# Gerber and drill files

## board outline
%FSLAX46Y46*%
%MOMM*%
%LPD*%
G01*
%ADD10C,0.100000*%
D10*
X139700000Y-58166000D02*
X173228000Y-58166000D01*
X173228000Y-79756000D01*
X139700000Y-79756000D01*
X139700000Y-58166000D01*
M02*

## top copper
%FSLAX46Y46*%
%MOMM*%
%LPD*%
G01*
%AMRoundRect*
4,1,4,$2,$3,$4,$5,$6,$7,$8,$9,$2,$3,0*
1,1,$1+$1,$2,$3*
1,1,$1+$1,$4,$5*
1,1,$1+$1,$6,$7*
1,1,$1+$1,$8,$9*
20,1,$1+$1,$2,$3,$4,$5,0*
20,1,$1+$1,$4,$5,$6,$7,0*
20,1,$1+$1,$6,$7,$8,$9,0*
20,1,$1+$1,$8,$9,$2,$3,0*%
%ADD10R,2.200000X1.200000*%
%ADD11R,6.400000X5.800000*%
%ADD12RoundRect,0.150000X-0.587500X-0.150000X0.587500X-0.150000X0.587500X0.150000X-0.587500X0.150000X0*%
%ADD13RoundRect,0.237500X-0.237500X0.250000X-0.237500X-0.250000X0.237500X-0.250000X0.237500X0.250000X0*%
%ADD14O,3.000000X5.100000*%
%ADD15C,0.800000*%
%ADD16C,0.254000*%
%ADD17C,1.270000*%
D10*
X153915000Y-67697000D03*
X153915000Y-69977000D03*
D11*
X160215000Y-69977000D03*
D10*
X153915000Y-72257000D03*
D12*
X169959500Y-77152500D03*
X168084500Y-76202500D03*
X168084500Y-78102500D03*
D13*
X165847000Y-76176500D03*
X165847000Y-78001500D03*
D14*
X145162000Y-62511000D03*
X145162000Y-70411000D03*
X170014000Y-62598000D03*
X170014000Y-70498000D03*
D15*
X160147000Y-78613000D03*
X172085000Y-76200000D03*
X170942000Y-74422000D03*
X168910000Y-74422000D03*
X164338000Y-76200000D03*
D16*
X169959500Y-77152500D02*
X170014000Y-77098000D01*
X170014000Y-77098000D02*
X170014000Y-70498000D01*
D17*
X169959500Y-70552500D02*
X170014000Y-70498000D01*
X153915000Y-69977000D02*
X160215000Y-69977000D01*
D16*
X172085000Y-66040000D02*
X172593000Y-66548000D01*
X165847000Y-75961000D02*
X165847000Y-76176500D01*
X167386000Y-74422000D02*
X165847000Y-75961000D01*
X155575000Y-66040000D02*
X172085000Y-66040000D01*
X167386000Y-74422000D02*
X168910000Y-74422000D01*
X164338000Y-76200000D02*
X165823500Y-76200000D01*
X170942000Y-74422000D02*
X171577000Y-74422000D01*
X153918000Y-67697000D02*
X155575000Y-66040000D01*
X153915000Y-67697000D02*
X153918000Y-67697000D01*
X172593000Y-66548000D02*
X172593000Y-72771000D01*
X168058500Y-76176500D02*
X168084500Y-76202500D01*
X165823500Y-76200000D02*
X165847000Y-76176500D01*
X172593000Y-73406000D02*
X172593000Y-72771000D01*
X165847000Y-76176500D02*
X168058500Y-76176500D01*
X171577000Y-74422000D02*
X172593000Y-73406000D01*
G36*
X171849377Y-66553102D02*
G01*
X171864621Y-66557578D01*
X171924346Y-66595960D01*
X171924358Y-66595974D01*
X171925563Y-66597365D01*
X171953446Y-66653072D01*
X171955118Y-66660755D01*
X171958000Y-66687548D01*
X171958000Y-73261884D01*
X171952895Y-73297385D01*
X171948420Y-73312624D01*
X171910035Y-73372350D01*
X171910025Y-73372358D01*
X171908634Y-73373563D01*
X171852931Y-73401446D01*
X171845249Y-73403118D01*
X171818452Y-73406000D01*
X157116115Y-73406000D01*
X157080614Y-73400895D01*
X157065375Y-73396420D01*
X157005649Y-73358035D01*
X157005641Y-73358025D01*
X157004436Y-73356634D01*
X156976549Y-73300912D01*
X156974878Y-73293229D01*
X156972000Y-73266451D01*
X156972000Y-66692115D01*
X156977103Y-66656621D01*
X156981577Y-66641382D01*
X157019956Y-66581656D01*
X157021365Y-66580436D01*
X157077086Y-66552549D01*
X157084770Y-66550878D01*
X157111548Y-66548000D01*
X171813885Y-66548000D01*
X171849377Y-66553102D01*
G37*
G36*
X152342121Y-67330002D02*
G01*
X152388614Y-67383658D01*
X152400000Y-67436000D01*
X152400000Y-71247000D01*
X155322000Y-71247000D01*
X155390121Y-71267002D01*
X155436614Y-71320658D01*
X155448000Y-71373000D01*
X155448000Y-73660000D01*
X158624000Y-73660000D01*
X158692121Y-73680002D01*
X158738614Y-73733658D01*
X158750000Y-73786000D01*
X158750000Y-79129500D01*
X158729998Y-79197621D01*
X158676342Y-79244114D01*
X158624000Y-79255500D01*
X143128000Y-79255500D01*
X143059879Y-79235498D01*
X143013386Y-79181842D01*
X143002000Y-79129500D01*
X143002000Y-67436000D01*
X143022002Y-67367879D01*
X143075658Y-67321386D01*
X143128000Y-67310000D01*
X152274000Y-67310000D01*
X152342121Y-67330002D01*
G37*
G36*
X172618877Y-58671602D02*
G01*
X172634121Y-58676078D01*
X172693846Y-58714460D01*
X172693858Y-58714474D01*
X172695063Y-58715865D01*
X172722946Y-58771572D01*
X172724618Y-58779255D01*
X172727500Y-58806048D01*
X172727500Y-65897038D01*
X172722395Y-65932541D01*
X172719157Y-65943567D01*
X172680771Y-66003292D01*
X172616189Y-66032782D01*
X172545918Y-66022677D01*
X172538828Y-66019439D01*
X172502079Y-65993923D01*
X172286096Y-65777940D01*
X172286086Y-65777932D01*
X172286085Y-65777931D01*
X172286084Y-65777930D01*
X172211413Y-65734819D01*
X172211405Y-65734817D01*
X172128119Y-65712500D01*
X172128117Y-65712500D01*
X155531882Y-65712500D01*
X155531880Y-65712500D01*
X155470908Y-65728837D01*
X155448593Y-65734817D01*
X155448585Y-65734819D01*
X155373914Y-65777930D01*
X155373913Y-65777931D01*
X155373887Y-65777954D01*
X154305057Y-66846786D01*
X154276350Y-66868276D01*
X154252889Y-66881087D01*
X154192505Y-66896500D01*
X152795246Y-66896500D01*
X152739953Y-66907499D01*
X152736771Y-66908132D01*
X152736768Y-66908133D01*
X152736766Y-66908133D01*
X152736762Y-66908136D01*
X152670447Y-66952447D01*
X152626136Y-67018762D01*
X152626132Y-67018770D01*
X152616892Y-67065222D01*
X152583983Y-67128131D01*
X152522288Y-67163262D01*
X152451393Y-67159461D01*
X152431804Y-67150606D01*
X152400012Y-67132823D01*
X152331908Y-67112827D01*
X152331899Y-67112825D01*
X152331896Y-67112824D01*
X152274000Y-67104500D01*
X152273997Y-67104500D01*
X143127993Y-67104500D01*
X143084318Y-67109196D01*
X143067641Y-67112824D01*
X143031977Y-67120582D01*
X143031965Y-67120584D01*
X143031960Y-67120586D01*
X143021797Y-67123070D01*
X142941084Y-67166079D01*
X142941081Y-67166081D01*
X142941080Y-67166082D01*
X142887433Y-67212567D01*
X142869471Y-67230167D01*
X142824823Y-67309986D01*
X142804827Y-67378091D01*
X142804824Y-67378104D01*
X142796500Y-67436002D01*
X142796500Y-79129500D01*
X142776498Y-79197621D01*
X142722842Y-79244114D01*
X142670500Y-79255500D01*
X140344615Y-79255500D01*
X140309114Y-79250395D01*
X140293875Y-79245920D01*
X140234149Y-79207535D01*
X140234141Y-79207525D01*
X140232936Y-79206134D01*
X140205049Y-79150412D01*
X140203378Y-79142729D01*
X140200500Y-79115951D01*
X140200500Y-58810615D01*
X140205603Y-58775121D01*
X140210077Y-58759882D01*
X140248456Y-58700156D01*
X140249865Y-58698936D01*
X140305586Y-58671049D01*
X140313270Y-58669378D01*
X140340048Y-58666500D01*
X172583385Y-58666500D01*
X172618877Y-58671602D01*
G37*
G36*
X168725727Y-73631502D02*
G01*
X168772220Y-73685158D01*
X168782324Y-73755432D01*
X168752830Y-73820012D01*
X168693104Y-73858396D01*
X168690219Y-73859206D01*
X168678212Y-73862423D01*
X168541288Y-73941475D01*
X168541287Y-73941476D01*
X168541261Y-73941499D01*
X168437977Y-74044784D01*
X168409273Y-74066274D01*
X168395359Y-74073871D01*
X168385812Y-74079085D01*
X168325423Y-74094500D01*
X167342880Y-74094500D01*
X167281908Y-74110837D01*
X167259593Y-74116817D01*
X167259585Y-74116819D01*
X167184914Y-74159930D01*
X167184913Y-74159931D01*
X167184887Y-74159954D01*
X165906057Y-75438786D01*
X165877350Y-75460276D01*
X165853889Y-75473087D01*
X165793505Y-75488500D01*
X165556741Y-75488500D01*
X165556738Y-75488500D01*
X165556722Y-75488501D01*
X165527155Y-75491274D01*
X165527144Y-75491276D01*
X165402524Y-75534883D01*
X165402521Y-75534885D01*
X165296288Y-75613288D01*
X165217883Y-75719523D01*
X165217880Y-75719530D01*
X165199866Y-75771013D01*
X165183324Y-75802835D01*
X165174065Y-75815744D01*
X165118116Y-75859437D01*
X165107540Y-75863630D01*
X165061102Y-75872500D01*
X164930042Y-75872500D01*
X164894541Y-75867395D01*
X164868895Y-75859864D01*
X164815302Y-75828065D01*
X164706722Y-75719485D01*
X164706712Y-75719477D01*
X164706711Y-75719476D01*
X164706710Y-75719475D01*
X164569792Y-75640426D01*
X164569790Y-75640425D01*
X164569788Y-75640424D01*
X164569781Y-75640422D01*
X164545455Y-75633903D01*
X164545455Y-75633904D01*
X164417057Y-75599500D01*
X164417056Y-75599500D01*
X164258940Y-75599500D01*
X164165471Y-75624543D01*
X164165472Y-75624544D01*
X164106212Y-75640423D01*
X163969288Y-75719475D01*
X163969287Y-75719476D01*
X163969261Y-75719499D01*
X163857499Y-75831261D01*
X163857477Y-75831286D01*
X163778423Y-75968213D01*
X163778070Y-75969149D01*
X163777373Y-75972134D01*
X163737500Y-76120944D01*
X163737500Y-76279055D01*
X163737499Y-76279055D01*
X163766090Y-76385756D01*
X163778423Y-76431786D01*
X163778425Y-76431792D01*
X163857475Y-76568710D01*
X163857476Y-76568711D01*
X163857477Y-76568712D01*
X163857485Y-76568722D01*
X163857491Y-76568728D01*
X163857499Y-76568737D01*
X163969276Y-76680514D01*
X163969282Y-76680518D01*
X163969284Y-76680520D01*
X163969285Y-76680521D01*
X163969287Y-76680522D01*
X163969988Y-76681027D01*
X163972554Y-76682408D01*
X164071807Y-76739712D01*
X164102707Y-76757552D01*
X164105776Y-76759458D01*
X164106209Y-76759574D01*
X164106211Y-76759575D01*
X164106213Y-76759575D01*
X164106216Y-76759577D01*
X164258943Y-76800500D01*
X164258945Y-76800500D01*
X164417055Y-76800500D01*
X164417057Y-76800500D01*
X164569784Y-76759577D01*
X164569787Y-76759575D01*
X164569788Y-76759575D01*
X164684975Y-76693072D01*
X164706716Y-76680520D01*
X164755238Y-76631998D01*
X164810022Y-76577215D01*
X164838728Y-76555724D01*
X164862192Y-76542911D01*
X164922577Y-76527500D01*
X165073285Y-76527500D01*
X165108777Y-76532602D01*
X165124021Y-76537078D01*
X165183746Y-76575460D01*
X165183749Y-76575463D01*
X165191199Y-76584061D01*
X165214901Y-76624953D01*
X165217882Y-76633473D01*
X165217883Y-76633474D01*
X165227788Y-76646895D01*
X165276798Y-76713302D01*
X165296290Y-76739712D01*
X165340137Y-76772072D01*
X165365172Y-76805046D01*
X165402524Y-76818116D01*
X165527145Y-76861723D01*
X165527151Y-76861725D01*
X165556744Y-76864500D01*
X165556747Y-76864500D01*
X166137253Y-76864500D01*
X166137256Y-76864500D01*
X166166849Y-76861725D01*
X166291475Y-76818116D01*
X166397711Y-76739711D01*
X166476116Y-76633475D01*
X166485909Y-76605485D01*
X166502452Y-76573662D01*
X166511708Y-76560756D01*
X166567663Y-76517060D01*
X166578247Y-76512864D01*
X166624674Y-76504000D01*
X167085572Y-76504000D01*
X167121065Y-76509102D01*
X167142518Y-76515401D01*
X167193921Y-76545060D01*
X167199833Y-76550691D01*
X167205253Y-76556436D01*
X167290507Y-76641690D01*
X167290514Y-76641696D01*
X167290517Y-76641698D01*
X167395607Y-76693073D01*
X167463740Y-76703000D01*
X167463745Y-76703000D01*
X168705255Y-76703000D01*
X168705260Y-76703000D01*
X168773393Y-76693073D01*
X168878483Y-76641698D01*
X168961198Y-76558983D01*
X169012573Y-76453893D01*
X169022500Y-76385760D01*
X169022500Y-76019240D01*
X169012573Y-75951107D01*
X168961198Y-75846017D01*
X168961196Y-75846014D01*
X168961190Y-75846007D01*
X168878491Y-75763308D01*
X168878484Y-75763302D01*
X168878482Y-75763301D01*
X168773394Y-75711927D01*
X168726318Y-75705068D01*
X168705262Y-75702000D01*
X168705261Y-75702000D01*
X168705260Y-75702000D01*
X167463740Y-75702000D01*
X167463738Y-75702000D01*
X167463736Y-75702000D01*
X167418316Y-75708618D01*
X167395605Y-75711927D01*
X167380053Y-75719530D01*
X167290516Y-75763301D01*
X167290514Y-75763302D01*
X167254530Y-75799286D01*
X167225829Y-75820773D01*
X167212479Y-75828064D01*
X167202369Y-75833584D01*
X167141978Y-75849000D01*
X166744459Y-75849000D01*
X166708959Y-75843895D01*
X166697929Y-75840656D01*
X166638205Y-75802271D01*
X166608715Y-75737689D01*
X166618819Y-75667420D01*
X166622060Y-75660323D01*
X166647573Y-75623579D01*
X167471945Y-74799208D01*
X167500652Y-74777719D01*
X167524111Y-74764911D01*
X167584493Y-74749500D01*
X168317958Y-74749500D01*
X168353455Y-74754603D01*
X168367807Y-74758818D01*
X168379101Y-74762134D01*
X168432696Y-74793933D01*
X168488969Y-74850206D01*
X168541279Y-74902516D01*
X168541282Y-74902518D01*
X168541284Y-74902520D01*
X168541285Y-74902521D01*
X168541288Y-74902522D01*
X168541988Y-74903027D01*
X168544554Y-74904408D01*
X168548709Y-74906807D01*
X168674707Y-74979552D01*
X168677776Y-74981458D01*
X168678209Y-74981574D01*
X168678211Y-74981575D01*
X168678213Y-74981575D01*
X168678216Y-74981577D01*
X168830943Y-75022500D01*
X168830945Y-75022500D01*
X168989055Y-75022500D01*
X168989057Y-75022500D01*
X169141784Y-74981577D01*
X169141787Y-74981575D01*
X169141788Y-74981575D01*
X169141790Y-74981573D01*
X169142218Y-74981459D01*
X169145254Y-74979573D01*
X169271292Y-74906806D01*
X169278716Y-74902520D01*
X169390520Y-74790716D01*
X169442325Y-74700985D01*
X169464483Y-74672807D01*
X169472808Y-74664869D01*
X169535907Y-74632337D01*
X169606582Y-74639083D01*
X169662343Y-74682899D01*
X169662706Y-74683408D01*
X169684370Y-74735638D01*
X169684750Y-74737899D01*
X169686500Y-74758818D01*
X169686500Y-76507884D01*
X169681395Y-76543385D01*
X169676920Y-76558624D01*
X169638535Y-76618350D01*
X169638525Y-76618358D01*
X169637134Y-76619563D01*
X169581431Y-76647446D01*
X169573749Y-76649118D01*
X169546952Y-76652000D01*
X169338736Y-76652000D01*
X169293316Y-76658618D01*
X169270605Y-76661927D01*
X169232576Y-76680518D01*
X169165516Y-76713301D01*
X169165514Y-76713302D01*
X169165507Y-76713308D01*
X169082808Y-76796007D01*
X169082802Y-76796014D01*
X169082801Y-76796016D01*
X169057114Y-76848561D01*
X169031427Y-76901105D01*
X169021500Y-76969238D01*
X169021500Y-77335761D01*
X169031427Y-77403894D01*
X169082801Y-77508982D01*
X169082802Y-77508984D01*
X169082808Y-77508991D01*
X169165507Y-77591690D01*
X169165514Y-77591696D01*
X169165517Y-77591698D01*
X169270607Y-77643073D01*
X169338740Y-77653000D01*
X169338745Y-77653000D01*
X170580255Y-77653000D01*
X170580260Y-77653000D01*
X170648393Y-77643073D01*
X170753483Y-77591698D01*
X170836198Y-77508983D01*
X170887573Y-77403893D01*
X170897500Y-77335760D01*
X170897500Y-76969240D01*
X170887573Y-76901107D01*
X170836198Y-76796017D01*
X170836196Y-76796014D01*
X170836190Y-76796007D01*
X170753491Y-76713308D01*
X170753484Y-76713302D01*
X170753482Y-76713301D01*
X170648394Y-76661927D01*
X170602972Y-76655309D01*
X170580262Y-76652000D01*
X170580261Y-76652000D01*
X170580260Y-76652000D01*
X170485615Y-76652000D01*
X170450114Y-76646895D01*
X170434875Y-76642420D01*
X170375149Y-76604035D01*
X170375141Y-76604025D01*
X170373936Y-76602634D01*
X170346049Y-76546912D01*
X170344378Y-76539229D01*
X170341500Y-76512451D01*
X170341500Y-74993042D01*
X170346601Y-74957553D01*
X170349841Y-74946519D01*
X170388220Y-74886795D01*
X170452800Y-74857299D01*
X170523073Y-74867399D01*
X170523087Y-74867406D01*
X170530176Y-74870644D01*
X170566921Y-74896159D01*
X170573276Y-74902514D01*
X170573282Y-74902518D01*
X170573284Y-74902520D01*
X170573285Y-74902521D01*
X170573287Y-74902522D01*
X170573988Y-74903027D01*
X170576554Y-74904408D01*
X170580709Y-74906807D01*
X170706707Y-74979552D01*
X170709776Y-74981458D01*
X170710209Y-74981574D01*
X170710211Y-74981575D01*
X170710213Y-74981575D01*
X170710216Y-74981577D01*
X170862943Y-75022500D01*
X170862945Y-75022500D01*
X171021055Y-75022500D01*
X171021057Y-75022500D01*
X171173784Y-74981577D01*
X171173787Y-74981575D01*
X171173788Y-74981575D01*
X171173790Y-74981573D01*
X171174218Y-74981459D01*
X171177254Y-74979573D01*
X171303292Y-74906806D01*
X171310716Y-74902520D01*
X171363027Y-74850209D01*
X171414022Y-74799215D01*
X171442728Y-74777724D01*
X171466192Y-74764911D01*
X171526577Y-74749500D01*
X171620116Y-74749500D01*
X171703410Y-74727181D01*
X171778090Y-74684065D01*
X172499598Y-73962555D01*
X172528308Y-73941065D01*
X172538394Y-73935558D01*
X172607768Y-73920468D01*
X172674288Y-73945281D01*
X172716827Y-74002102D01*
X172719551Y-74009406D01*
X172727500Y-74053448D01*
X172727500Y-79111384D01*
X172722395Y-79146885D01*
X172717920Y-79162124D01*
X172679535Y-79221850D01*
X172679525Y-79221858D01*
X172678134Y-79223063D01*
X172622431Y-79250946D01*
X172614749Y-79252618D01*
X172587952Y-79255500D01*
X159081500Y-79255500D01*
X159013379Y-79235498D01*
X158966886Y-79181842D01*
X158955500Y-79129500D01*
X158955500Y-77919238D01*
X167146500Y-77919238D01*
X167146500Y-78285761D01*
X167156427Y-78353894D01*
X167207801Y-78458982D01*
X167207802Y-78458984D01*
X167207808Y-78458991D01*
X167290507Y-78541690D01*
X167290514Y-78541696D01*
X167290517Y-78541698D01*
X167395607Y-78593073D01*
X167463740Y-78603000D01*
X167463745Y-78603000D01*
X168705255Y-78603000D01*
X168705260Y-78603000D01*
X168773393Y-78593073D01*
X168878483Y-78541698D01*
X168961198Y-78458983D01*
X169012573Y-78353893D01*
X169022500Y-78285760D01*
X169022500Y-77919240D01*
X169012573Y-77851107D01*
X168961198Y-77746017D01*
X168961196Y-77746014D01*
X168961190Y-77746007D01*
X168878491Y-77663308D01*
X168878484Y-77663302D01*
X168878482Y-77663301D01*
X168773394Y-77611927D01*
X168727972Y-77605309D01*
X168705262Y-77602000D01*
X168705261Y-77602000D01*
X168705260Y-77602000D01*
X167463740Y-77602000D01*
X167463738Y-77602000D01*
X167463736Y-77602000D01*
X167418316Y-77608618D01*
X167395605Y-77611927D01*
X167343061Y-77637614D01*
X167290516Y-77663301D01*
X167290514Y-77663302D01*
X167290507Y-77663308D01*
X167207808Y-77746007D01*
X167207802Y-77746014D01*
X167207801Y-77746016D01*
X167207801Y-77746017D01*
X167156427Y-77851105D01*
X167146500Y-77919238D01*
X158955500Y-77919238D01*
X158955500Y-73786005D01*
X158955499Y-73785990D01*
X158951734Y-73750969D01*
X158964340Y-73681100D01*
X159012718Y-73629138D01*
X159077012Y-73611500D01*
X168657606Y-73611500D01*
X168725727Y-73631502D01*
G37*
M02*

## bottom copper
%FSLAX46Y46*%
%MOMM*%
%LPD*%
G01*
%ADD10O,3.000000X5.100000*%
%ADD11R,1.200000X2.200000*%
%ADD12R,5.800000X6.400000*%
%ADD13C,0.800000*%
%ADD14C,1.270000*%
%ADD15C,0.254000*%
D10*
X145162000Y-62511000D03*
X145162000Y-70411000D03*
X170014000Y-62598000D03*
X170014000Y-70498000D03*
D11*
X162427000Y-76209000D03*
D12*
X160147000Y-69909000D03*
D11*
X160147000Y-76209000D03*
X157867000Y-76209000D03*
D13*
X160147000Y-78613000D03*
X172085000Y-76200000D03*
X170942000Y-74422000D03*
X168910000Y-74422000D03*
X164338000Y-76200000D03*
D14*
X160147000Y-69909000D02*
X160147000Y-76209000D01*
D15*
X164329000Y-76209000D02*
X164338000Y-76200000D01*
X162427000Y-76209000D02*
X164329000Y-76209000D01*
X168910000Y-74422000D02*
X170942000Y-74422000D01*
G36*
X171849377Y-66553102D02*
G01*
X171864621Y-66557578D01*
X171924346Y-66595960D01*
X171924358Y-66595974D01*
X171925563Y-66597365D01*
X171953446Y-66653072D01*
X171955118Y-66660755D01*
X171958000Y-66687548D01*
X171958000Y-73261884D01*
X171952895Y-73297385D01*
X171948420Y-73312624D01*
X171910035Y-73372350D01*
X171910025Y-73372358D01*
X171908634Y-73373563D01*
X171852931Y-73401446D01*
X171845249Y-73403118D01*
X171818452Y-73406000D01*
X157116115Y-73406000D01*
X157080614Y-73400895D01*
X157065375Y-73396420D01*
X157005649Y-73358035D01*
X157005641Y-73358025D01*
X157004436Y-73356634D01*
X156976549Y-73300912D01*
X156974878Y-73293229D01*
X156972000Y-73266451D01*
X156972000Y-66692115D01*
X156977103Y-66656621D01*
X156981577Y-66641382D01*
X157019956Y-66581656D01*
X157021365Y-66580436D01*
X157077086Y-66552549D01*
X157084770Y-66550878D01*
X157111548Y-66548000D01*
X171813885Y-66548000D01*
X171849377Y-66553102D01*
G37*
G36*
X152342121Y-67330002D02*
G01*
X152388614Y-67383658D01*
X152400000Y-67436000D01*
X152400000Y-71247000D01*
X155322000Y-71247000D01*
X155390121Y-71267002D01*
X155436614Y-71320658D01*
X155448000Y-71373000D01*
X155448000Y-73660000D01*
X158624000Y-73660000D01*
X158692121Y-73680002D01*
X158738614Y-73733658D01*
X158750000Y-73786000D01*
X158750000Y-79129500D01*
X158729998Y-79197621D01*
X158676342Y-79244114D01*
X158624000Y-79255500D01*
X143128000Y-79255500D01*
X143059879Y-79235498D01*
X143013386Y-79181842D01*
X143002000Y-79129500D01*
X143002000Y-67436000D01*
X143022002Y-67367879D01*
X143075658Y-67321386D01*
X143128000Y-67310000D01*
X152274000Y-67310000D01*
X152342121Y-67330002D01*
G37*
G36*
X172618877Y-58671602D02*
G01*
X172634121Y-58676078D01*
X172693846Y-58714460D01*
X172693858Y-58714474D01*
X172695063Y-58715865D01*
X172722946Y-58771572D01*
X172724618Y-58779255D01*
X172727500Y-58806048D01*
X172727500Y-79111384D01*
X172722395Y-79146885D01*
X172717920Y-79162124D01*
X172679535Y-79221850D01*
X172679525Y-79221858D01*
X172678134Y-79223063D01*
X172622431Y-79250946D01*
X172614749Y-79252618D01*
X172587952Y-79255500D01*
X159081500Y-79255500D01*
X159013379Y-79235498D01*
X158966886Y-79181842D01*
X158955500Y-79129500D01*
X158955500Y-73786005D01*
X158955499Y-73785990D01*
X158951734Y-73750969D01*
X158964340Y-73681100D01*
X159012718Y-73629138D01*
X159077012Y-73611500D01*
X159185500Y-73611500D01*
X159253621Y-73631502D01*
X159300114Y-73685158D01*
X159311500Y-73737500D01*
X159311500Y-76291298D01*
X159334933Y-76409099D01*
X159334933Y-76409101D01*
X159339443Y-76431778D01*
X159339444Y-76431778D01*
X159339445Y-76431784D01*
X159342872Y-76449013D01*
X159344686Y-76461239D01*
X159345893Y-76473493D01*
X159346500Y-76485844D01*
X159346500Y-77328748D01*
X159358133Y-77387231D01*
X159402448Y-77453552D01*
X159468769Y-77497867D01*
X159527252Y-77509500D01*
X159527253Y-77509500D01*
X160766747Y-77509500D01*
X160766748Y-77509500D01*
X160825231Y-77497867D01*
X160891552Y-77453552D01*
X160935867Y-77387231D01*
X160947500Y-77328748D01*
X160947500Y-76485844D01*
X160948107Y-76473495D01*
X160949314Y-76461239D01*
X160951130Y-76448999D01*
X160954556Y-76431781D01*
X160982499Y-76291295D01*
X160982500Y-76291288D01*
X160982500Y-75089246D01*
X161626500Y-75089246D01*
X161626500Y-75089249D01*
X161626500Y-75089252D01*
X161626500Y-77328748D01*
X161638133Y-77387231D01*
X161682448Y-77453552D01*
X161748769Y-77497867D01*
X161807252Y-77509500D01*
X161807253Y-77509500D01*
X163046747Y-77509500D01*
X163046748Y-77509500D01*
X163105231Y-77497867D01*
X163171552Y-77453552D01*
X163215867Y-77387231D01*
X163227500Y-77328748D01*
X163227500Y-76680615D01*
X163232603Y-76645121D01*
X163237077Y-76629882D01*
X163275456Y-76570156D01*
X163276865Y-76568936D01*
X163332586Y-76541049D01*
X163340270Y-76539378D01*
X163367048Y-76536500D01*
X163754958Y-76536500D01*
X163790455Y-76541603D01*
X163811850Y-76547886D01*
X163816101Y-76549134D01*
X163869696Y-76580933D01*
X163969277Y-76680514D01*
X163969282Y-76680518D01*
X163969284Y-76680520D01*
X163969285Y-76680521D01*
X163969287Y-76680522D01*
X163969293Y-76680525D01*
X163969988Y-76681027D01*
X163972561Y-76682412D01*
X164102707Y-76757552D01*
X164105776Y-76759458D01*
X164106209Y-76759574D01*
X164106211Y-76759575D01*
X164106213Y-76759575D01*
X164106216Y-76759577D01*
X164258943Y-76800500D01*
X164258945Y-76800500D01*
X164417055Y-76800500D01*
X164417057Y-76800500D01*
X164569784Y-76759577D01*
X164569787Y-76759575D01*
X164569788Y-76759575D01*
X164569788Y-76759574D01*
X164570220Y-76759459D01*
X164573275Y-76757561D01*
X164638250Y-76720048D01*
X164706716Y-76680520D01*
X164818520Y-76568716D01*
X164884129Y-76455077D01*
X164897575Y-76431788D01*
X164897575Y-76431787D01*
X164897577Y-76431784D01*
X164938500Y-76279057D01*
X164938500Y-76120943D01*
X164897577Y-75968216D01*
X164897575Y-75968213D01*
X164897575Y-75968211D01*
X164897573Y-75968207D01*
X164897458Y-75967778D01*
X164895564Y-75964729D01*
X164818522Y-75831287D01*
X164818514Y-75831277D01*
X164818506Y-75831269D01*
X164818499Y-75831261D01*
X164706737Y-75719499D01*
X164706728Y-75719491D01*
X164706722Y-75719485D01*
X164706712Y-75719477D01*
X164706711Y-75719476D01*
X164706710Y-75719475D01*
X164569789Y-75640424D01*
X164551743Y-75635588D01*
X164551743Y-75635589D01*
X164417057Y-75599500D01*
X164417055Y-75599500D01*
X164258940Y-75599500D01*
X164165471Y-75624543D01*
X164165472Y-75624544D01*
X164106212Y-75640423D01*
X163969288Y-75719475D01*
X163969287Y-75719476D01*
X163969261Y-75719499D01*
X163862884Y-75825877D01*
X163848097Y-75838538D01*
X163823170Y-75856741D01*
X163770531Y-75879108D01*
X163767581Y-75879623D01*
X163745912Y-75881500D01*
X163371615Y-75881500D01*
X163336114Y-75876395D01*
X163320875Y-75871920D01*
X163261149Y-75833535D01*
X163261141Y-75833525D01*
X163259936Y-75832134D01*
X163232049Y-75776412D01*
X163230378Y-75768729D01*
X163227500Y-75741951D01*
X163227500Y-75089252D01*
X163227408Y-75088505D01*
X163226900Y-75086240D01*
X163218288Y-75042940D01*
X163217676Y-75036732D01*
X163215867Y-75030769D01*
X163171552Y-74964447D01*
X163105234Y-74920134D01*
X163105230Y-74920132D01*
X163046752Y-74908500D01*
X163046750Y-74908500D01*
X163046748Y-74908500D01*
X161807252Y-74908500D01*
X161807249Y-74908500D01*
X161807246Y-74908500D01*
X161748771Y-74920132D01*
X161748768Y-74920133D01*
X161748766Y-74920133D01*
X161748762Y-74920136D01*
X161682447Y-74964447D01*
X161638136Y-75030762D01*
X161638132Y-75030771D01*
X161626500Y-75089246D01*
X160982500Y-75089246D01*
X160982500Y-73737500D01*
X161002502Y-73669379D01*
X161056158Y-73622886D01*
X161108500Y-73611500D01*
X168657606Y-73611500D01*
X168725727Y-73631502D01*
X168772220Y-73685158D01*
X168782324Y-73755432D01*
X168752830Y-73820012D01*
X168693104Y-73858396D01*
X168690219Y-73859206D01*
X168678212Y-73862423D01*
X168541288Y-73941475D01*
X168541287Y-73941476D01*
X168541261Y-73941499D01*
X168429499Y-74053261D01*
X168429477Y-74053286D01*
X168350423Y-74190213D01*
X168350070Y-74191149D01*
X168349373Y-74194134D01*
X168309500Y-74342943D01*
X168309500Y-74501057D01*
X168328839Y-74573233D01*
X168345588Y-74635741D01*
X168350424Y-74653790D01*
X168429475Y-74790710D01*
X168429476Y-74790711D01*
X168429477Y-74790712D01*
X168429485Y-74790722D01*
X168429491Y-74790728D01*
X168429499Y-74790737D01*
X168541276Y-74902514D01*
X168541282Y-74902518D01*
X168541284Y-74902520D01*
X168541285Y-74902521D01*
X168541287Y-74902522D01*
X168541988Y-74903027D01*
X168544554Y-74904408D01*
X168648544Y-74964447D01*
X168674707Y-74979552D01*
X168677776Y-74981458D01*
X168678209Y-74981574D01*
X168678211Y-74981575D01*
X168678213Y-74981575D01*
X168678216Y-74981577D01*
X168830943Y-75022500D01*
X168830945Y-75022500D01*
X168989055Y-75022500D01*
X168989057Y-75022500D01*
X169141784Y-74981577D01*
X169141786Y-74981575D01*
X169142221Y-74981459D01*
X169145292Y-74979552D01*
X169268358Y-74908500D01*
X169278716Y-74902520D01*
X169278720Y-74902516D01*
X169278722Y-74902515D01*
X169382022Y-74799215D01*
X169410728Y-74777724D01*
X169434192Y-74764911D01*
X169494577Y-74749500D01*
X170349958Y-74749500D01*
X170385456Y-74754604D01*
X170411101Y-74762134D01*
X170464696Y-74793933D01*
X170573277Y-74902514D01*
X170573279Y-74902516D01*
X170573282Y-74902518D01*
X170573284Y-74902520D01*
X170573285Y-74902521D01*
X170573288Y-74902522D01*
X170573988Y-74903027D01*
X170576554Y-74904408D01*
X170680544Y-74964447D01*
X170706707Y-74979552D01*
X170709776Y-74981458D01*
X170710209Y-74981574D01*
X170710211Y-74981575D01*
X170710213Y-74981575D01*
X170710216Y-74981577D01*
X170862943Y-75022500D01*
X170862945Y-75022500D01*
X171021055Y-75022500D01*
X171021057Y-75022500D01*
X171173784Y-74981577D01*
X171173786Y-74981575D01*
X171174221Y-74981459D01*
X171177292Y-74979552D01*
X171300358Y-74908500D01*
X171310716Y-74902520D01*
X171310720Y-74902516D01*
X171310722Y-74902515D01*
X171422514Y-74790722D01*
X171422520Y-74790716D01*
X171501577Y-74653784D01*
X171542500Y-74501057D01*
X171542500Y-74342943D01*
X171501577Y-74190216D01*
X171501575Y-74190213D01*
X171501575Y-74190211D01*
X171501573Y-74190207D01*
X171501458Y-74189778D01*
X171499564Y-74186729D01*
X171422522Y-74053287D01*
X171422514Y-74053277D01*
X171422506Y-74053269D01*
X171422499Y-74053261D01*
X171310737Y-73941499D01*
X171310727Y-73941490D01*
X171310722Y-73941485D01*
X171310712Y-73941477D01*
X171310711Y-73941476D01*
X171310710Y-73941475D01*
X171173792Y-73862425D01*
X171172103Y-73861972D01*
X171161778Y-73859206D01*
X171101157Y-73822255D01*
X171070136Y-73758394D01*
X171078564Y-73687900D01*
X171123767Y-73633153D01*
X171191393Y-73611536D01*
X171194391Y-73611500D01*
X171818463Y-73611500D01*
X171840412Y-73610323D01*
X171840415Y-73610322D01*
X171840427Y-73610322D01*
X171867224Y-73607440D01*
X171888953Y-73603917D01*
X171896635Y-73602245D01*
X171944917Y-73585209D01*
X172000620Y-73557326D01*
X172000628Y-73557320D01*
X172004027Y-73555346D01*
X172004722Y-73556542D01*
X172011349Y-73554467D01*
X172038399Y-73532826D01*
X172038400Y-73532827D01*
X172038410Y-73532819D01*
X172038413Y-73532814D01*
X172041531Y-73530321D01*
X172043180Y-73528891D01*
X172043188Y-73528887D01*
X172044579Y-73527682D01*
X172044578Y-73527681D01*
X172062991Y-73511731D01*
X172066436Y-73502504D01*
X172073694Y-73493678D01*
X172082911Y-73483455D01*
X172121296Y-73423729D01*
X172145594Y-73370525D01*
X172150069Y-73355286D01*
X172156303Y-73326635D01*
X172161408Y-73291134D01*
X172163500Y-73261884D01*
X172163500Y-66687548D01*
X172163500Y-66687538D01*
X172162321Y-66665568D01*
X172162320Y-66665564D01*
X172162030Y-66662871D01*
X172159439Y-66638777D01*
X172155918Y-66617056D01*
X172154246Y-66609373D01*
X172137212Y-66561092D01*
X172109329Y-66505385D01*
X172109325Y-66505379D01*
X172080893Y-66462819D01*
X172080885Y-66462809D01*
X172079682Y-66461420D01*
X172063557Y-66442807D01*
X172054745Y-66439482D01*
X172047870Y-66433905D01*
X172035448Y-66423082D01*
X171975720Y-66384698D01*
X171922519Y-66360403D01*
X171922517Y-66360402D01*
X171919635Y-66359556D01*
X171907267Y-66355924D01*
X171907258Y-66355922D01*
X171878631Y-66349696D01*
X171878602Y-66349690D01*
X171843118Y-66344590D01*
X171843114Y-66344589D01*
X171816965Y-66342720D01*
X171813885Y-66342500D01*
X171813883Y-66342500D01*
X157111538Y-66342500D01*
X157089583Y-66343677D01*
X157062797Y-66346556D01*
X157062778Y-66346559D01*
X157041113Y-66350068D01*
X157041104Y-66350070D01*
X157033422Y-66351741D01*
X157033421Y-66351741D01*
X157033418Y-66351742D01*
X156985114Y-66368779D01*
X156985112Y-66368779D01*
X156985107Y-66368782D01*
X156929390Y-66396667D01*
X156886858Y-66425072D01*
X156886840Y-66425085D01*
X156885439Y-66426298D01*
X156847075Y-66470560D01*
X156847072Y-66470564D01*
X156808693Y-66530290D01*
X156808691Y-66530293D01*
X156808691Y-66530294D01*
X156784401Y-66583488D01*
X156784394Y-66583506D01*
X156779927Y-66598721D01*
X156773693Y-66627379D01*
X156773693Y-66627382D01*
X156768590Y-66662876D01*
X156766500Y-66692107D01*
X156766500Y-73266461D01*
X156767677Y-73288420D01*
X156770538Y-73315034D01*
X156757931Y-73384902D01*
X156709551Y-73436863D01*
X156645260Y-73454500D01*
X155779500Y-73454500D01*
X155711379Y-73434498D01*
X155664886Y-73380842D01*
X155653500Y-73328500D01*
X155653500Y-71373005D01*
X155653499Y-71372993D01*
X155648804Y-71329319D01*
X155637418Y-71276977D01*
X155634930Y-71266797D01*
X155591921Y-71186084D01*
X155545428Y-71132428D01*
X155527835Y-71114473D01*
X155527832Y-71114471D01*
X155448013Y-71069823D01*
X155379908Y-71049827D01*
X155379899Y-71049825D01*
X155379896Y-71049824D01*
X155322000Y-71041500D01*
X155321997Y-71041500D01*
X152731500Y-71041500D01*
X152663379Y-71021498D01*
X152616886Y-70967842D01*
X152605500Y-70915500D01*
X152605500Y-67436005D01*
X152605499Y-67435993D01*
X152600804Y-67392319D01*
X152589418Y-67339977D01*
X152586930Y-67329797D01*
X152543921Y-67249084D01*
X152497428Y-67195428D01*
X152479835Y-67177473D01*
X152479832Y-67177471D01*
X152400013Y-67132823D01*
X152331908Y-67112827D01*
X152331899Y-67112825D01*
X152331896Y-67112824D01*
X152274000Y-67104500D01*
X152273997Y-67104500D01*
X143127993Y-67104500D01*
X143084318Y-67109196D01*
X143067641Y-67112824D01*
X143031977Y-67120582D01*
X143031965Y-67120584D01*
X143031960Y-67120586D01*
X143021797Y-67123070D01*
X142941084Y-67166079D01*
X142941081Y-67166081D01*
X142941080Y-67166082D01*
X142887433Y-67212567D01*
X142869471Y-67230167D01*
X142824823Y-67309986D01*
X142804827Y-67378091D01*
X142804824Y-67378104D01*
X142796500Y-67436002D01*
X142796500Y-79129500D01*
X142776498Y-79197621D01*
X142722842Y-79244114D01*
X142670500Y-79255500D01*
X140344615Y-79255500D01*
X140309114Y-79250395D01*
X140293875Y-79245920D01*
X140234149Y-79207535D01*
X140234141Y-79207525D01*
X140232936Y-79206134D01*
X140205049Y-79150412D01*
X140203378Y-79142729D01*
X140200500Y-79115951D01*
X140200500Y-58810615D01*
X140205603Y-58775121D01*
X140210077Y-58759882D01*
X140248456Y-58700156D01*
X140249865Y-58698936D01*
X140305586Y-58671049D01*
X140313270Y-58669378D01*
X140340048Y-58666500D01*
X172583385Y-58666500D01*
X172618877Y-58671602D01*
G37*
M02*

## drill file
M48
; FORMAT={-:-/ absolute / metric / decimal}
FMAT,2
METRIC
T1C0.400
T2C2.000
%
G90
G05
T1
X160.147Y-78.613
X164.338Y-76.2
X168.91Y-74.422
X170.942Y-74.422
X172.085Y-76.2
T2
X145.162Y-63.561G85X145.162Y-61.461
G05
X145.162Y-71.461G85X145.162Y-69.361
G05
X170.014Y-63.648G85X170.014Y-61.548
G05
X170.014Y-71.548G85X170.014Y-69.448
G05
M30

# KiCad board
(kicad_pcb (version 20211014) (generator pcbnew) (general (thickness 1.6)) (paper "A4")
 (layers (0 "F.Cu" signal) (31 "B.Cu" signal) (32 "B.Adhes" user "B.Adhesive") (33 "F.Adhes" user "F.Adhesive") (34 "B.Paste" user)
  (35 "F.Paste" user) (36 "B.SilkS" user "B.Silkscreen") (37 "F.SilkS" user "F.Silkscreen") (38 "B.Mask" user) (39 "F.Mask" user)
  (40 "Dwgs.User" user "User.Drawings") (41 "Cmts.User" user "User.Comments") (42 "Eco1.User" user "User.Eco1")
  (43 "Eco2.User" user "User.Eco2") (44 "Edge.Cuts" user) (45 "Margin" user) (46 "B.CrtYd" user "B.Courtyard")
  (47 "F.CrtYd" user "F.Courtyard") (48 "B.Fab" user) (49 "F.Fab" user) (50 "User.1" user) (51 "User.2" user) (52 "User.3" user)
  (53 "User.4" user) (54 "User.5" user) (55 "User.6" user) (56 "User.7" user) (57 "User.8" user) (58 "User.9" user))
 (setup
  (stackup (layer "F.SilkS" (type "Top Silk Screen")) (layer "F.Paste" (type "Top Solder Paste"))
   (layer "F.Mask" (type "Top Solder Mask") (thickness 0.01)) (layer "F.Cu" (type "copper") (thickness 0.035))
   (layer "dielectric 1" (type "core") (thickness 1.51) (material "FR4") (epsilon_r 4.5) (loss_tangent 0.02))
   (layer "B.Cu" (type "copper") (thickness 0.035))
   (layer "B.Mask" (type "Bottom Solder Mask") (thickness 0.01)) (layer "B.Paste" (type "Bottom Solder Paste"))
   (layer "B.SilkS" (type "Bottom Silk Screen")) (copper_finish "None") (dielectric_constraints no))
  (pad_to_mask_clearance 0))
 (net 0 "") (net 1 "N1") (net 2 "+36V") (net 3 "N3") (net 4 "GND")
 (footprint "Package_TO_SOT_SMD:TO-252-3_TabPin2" (layer "F.Cu") (at 158.115 69.977)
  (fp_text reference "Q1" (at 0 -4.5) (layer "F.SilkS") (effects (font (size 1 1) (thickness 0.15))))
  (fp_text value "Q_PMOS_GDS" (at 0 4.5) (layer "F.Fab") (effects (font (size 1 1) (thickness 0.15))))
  (pad "" smd rect (at 0.425 1.525) (size 3.05 2.75) (layers "F.Paste"))
  (pad "" smd rect (at 3.775 1.525) (size 3.05 2.75) (layers "F.Paste"))
  (pad "" smd rect (at 3.775 -1.525) (size 3.05 2.75) (layers "F.Paste"))
  (pad "" smd rect (at 0.425 -1.525) (size 3.05 2.75) (layers "F.Paste"))
  (pad "1" smd rect (at -4.2 -2.28) (size 2.2 1.2) (layers "F.Cu" "F.Paste" "F.Mask") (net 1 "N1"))
  (pad "2" smd rect (at -4.2 0) (size 2.2 1.2) (layers "F.Cu" "F.Paste" "F.Mask") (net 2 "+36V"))
  (pad "2" smd rect (at 2.1 0) (size 6.4 5.8) (layers "F.Cu" "F.Mask") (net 2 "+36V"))
  (pad "3" smd rect (at -4.2 2.28) (size 2.2 1.2) (layers "F.Cu" "F.Paste" "F.Mask") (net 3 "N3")))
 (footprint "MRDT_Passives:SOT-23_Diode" (layer "F.Cu") (at 169.672 75.0425)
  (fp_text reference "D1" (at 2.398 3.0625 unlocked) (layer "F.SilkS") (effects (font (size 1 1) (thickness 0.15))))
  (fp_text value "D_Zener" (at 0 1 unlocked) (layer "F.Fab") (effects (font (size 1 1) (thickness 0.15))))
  (pad "1" smd roundrect (at 0.2875 2.11) (size 1.475 0.6) (layers "F.Cu" "F.Paste" "F.Mask") (roundrect_rratio 0.25) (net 2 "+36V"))
  (pad "2" smd roundrect (at -1.5875 1.16) (size 1.475 0.6) (layers "F.Cu" "F.Paste" "F.Mask") (roundrect_rratio 0.25) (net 1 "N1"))
  (pad "3" smd roundrect (at -1.5875 3.06) (size 1.475 0.6) (layers "F.Cu" "F.Paste" "F.Mask") (roundrect_rratio 0.25)))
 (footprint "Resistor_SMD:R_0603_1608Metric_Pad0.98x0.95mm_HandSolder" (layer "F.Cu") (at 165.847 77.089 -90)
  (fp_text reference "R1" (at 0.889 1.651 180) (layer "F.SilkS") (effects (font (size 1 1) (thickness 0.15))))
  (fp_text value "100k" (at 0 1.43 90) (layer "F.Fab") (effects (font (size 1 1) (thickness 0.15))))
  (pad "1" smd roundrect (at -0.9125 0 270) (size 0.975 0.95) (layers "F.Cu" "F.Paste" "F.Mask") (roundrect_rratio 0.25) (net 1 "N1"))
  (pad "2" smd roundrect (at 0.9125 0 270) (size 0.975 0.95) (layers "F.Cu" "F.Paste" "F.Mask") (roundrect_rratio 0.25) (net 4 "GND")))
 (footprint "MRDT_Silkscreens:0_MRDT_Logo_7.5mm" (layer "F.Cu") (at 155.829 62.357)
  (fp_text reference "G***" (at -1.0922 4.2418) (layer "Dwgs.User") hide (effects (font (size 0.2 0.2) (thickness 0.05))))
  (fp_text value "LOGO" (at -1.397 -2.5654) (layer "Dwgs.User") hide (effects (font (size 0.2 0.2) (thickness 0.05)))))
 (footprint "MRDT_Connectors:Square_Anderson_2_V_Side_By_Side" (layer "F.Cu") (at 145.288 66.548 -90)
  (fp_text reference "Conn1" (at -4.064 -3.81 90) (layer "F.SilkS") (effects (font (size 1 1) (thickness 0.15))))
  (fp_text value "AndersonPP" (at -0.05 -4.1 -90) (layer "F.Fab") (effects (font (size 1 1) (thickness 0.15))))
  (pad "1" thru_hole oval locked (at -4.037 0.126 180) (size 3 5.1) (drill oval 2 4.1) (layers F&B.Cu *.Mask) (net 4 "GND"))
  (pad "2" thru_hole oval locked (at 3.863 0.126 180) (size 3 5.1) (drill oval 2 4.1) (layers F&B.Cu *.Mask) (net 3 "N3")))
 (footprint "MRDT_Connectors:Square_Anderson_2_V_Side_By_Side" (layer "F.Cu") (at 170.14 66.635 -90)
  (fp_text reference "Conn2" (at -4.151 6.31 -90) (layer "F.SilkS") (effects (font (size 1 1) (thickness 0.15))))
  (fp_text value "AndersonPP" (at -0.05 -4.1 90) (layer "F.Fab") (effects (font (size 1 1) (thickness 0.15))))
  (pad "1" thru_hole oval locked (at -4.037 0.126 180) (size 3 5.1) (drill oval 2 4.1) (layers F&B.Cu *.Mask) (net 4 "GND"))
  (pad "2" thru_hole oval locked (at 3.863 0.126 180) (size 3 5.1) (drill oval 2 4.1) (layers F&B.Cu *.Mask) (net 2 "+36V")))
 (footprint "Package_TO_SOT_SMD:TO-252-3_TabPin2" (layer "B.Cu") (at 160.147 72.009 90)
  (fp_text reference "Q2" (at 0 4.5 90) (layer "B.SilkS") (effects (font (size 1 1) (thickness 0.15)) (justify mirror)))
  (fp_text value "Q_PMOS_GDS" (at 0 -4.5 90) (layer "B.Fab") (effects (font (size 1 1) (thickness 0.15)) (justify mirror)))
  (pad "" smd rect (at 3.775 1.525 90) (size 3.05 2.75) (layers "B.Paste"))
  (pad "" smd rect (at 0.425 -1.525 90) (size 3.05 2.75) (layers "B.Paste"))
  (pad "" smd rect (at 0.425 1.525 90) (size 3.05 2.75) (layers "B.Paste"))
  (pad "" smd rect (at 3.775 -1.525 90) (size 3.05 2.75) (layers "B.Paste"))
  (pad "1" smd rect (at -4.2 2.28 90) (size 2.2 1.2) (layers "B.Cu" "B.Paste" "B.Mask") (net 1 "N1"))
  (pad "2" smd rect (at 2.1 0 90) (size 6.4 5.8) (layers "B.Cu" "B.Mask") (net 2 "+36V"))
  (pad "2" smd rect (at -4.2 0 90) (size 2.2 1.2) (layers "B.Cu" "B.Paste" "B.Mask") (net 2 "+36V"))
  (pad "3" smd rect (at -4.2 -2.28 90) (size 2.2 1.2) (layers "B.Cu" "B.Paste" "B.Mask") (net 3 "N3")))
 (gr_rect (start 139.7 58.166) (end 173.228 79.756) (layer "Edge.Cuts") (width 0.1) (fill none))
 (via (at 160.147 78.613) (size 0.8) (drill 0.4) (layers "F.Cu" "B.Cu") (free) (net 4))
 (via (at 172.085 76.2) (size 0.8) (drill 0.4) (layers "F.Cu" "B.Cu") (free) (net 4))
 (segment (start 169.9595 77.1525) (end 170.014 77.098) (width 0.254) (layer "F.Cu") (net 2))
 (segment (start 170.014 77.098) (end 170.014 70.498) (width 0.254) (layer "F.Cu") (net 2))
 (segment (start 169.9595 70.5525) (end 170.014 70.498) (width 1.27) (layer "F.Cu") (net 2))
 (segment (start 153.915 69.977) (end 160.215 69.977) (width 1.27) (layer "F.Cu") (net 2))
 (segment (start 160.147 69.909) (end 160.147 76.209) (width 1.27) (layer "B.Cu") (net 2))
 (segment (start 172.085 66.04) (end 172.593 66.548) (width 0.254) (layer "F.Cu") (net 1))
 (segment (start 165.847 75.961) (end 165.847 76.1765) (width 0.254) (layer "F.Cu") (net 1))
 (segment (start 167.386 74.422) (end 165.847 75.961) (width 0.254) (layer "F.Cu") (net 1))
 (segment (start 155.575 66.04) (end 172.085 66.04) (width 0.254) (layer "F.Cu") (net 1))
 (segment (start 167.386 74.422) (end 168.91 74.422) (width 0.254) (layer "F.Cu") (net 1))
 (segment (start 164.338 76.2) (end 165.8235 76.2) (width 0.254) (layer "F.Cu") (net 1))
 (segment (start 170.942 74.422) (end 171.577 74.422) (width 0.254) (layer "F.Cu") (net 1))
 (segment (start 153.918 67.697) (end 155.575 66.04) (width 0.254) (layer "F.Cu") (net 1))
 (segment (start 153.915 67.697) (end 153.918 67.697) (width 0.254) (layer "F.Cu") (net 1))
 (segment (start 172.593 66.548) (end 172.593 72.771) (width 0.254) (layer "F.Cu") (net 1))
 (segment (start 168.0585 76.1765) (end 168.0845 76.2025) (width 0.254) (layer "F.Cu") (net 1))
 (segment (start 165.8235 76.2) (end 165.847 76.1765) (width 0.254) (layer "F.Cu") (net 1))
 (segment (start 172.593 73.406) (end 172.593 72.771) (width 0.254) (layer "F.Cu") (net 1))
 (segment (start 165.847 76.1765) (end 168.0585 76.1765) (width 0.254) (layer "F.Cu") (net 1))
 (segment (start 171.577 74.422) (end 172.593 73.406) (width 0.254) (layer "F.Cu") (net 1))
 (via (at 170.942 74.422) (size 0.8) (drill 0.4) (layers "F.Cu" "B.Cu") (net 1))
 (via (at 168.91 74.422) (size 0.8) (drill 0.4) (layers "F.Cu" "B.Cu") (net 1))
 (via (at 164.338 76.2) (size 0.8) (drill 0.4) (layers "F.Cu" "B.Cu") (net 1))
 (segment (start 164.329 76.209) (end 164.338 76.2) (width 0.254) (layer "B.Cu") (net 1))
 (segment (start 162.427 76.209) (end 164.329 76.209) (width 0.254) (layer "B.Cu") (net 1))
 (segment (start 168.91 74.422) (end 170.942 74.422) (width 0.254) (layer "B.Cu") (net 1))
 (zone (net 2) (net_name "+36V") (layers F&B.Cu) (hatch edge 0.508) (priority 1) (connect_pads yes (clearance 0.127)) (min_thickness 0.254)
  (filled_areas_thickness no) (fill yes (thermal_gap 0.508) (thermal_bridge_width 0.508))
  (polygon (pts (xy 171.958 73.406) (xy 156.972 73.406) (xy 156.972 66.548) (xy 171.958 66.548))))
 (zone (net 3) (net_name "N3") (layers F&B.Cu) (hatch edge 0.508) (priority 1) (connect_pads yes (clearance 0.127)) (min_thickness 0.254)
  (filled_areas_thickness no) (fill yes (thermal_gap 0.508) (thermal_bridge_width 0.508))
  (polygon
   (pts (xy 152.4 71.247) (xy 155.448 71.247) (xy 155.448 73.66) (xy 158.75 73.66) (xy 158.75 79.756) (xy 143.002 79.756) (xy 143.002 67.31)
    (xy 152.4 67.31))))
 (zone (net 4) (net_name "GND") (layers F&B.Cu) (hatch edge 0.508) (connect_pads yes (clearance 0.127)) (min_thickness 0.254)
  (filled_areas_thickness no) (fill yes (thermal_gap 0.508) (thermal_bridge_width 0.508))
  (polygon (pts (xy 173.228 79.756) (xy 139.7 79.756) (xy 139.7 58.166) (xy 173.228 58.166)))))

